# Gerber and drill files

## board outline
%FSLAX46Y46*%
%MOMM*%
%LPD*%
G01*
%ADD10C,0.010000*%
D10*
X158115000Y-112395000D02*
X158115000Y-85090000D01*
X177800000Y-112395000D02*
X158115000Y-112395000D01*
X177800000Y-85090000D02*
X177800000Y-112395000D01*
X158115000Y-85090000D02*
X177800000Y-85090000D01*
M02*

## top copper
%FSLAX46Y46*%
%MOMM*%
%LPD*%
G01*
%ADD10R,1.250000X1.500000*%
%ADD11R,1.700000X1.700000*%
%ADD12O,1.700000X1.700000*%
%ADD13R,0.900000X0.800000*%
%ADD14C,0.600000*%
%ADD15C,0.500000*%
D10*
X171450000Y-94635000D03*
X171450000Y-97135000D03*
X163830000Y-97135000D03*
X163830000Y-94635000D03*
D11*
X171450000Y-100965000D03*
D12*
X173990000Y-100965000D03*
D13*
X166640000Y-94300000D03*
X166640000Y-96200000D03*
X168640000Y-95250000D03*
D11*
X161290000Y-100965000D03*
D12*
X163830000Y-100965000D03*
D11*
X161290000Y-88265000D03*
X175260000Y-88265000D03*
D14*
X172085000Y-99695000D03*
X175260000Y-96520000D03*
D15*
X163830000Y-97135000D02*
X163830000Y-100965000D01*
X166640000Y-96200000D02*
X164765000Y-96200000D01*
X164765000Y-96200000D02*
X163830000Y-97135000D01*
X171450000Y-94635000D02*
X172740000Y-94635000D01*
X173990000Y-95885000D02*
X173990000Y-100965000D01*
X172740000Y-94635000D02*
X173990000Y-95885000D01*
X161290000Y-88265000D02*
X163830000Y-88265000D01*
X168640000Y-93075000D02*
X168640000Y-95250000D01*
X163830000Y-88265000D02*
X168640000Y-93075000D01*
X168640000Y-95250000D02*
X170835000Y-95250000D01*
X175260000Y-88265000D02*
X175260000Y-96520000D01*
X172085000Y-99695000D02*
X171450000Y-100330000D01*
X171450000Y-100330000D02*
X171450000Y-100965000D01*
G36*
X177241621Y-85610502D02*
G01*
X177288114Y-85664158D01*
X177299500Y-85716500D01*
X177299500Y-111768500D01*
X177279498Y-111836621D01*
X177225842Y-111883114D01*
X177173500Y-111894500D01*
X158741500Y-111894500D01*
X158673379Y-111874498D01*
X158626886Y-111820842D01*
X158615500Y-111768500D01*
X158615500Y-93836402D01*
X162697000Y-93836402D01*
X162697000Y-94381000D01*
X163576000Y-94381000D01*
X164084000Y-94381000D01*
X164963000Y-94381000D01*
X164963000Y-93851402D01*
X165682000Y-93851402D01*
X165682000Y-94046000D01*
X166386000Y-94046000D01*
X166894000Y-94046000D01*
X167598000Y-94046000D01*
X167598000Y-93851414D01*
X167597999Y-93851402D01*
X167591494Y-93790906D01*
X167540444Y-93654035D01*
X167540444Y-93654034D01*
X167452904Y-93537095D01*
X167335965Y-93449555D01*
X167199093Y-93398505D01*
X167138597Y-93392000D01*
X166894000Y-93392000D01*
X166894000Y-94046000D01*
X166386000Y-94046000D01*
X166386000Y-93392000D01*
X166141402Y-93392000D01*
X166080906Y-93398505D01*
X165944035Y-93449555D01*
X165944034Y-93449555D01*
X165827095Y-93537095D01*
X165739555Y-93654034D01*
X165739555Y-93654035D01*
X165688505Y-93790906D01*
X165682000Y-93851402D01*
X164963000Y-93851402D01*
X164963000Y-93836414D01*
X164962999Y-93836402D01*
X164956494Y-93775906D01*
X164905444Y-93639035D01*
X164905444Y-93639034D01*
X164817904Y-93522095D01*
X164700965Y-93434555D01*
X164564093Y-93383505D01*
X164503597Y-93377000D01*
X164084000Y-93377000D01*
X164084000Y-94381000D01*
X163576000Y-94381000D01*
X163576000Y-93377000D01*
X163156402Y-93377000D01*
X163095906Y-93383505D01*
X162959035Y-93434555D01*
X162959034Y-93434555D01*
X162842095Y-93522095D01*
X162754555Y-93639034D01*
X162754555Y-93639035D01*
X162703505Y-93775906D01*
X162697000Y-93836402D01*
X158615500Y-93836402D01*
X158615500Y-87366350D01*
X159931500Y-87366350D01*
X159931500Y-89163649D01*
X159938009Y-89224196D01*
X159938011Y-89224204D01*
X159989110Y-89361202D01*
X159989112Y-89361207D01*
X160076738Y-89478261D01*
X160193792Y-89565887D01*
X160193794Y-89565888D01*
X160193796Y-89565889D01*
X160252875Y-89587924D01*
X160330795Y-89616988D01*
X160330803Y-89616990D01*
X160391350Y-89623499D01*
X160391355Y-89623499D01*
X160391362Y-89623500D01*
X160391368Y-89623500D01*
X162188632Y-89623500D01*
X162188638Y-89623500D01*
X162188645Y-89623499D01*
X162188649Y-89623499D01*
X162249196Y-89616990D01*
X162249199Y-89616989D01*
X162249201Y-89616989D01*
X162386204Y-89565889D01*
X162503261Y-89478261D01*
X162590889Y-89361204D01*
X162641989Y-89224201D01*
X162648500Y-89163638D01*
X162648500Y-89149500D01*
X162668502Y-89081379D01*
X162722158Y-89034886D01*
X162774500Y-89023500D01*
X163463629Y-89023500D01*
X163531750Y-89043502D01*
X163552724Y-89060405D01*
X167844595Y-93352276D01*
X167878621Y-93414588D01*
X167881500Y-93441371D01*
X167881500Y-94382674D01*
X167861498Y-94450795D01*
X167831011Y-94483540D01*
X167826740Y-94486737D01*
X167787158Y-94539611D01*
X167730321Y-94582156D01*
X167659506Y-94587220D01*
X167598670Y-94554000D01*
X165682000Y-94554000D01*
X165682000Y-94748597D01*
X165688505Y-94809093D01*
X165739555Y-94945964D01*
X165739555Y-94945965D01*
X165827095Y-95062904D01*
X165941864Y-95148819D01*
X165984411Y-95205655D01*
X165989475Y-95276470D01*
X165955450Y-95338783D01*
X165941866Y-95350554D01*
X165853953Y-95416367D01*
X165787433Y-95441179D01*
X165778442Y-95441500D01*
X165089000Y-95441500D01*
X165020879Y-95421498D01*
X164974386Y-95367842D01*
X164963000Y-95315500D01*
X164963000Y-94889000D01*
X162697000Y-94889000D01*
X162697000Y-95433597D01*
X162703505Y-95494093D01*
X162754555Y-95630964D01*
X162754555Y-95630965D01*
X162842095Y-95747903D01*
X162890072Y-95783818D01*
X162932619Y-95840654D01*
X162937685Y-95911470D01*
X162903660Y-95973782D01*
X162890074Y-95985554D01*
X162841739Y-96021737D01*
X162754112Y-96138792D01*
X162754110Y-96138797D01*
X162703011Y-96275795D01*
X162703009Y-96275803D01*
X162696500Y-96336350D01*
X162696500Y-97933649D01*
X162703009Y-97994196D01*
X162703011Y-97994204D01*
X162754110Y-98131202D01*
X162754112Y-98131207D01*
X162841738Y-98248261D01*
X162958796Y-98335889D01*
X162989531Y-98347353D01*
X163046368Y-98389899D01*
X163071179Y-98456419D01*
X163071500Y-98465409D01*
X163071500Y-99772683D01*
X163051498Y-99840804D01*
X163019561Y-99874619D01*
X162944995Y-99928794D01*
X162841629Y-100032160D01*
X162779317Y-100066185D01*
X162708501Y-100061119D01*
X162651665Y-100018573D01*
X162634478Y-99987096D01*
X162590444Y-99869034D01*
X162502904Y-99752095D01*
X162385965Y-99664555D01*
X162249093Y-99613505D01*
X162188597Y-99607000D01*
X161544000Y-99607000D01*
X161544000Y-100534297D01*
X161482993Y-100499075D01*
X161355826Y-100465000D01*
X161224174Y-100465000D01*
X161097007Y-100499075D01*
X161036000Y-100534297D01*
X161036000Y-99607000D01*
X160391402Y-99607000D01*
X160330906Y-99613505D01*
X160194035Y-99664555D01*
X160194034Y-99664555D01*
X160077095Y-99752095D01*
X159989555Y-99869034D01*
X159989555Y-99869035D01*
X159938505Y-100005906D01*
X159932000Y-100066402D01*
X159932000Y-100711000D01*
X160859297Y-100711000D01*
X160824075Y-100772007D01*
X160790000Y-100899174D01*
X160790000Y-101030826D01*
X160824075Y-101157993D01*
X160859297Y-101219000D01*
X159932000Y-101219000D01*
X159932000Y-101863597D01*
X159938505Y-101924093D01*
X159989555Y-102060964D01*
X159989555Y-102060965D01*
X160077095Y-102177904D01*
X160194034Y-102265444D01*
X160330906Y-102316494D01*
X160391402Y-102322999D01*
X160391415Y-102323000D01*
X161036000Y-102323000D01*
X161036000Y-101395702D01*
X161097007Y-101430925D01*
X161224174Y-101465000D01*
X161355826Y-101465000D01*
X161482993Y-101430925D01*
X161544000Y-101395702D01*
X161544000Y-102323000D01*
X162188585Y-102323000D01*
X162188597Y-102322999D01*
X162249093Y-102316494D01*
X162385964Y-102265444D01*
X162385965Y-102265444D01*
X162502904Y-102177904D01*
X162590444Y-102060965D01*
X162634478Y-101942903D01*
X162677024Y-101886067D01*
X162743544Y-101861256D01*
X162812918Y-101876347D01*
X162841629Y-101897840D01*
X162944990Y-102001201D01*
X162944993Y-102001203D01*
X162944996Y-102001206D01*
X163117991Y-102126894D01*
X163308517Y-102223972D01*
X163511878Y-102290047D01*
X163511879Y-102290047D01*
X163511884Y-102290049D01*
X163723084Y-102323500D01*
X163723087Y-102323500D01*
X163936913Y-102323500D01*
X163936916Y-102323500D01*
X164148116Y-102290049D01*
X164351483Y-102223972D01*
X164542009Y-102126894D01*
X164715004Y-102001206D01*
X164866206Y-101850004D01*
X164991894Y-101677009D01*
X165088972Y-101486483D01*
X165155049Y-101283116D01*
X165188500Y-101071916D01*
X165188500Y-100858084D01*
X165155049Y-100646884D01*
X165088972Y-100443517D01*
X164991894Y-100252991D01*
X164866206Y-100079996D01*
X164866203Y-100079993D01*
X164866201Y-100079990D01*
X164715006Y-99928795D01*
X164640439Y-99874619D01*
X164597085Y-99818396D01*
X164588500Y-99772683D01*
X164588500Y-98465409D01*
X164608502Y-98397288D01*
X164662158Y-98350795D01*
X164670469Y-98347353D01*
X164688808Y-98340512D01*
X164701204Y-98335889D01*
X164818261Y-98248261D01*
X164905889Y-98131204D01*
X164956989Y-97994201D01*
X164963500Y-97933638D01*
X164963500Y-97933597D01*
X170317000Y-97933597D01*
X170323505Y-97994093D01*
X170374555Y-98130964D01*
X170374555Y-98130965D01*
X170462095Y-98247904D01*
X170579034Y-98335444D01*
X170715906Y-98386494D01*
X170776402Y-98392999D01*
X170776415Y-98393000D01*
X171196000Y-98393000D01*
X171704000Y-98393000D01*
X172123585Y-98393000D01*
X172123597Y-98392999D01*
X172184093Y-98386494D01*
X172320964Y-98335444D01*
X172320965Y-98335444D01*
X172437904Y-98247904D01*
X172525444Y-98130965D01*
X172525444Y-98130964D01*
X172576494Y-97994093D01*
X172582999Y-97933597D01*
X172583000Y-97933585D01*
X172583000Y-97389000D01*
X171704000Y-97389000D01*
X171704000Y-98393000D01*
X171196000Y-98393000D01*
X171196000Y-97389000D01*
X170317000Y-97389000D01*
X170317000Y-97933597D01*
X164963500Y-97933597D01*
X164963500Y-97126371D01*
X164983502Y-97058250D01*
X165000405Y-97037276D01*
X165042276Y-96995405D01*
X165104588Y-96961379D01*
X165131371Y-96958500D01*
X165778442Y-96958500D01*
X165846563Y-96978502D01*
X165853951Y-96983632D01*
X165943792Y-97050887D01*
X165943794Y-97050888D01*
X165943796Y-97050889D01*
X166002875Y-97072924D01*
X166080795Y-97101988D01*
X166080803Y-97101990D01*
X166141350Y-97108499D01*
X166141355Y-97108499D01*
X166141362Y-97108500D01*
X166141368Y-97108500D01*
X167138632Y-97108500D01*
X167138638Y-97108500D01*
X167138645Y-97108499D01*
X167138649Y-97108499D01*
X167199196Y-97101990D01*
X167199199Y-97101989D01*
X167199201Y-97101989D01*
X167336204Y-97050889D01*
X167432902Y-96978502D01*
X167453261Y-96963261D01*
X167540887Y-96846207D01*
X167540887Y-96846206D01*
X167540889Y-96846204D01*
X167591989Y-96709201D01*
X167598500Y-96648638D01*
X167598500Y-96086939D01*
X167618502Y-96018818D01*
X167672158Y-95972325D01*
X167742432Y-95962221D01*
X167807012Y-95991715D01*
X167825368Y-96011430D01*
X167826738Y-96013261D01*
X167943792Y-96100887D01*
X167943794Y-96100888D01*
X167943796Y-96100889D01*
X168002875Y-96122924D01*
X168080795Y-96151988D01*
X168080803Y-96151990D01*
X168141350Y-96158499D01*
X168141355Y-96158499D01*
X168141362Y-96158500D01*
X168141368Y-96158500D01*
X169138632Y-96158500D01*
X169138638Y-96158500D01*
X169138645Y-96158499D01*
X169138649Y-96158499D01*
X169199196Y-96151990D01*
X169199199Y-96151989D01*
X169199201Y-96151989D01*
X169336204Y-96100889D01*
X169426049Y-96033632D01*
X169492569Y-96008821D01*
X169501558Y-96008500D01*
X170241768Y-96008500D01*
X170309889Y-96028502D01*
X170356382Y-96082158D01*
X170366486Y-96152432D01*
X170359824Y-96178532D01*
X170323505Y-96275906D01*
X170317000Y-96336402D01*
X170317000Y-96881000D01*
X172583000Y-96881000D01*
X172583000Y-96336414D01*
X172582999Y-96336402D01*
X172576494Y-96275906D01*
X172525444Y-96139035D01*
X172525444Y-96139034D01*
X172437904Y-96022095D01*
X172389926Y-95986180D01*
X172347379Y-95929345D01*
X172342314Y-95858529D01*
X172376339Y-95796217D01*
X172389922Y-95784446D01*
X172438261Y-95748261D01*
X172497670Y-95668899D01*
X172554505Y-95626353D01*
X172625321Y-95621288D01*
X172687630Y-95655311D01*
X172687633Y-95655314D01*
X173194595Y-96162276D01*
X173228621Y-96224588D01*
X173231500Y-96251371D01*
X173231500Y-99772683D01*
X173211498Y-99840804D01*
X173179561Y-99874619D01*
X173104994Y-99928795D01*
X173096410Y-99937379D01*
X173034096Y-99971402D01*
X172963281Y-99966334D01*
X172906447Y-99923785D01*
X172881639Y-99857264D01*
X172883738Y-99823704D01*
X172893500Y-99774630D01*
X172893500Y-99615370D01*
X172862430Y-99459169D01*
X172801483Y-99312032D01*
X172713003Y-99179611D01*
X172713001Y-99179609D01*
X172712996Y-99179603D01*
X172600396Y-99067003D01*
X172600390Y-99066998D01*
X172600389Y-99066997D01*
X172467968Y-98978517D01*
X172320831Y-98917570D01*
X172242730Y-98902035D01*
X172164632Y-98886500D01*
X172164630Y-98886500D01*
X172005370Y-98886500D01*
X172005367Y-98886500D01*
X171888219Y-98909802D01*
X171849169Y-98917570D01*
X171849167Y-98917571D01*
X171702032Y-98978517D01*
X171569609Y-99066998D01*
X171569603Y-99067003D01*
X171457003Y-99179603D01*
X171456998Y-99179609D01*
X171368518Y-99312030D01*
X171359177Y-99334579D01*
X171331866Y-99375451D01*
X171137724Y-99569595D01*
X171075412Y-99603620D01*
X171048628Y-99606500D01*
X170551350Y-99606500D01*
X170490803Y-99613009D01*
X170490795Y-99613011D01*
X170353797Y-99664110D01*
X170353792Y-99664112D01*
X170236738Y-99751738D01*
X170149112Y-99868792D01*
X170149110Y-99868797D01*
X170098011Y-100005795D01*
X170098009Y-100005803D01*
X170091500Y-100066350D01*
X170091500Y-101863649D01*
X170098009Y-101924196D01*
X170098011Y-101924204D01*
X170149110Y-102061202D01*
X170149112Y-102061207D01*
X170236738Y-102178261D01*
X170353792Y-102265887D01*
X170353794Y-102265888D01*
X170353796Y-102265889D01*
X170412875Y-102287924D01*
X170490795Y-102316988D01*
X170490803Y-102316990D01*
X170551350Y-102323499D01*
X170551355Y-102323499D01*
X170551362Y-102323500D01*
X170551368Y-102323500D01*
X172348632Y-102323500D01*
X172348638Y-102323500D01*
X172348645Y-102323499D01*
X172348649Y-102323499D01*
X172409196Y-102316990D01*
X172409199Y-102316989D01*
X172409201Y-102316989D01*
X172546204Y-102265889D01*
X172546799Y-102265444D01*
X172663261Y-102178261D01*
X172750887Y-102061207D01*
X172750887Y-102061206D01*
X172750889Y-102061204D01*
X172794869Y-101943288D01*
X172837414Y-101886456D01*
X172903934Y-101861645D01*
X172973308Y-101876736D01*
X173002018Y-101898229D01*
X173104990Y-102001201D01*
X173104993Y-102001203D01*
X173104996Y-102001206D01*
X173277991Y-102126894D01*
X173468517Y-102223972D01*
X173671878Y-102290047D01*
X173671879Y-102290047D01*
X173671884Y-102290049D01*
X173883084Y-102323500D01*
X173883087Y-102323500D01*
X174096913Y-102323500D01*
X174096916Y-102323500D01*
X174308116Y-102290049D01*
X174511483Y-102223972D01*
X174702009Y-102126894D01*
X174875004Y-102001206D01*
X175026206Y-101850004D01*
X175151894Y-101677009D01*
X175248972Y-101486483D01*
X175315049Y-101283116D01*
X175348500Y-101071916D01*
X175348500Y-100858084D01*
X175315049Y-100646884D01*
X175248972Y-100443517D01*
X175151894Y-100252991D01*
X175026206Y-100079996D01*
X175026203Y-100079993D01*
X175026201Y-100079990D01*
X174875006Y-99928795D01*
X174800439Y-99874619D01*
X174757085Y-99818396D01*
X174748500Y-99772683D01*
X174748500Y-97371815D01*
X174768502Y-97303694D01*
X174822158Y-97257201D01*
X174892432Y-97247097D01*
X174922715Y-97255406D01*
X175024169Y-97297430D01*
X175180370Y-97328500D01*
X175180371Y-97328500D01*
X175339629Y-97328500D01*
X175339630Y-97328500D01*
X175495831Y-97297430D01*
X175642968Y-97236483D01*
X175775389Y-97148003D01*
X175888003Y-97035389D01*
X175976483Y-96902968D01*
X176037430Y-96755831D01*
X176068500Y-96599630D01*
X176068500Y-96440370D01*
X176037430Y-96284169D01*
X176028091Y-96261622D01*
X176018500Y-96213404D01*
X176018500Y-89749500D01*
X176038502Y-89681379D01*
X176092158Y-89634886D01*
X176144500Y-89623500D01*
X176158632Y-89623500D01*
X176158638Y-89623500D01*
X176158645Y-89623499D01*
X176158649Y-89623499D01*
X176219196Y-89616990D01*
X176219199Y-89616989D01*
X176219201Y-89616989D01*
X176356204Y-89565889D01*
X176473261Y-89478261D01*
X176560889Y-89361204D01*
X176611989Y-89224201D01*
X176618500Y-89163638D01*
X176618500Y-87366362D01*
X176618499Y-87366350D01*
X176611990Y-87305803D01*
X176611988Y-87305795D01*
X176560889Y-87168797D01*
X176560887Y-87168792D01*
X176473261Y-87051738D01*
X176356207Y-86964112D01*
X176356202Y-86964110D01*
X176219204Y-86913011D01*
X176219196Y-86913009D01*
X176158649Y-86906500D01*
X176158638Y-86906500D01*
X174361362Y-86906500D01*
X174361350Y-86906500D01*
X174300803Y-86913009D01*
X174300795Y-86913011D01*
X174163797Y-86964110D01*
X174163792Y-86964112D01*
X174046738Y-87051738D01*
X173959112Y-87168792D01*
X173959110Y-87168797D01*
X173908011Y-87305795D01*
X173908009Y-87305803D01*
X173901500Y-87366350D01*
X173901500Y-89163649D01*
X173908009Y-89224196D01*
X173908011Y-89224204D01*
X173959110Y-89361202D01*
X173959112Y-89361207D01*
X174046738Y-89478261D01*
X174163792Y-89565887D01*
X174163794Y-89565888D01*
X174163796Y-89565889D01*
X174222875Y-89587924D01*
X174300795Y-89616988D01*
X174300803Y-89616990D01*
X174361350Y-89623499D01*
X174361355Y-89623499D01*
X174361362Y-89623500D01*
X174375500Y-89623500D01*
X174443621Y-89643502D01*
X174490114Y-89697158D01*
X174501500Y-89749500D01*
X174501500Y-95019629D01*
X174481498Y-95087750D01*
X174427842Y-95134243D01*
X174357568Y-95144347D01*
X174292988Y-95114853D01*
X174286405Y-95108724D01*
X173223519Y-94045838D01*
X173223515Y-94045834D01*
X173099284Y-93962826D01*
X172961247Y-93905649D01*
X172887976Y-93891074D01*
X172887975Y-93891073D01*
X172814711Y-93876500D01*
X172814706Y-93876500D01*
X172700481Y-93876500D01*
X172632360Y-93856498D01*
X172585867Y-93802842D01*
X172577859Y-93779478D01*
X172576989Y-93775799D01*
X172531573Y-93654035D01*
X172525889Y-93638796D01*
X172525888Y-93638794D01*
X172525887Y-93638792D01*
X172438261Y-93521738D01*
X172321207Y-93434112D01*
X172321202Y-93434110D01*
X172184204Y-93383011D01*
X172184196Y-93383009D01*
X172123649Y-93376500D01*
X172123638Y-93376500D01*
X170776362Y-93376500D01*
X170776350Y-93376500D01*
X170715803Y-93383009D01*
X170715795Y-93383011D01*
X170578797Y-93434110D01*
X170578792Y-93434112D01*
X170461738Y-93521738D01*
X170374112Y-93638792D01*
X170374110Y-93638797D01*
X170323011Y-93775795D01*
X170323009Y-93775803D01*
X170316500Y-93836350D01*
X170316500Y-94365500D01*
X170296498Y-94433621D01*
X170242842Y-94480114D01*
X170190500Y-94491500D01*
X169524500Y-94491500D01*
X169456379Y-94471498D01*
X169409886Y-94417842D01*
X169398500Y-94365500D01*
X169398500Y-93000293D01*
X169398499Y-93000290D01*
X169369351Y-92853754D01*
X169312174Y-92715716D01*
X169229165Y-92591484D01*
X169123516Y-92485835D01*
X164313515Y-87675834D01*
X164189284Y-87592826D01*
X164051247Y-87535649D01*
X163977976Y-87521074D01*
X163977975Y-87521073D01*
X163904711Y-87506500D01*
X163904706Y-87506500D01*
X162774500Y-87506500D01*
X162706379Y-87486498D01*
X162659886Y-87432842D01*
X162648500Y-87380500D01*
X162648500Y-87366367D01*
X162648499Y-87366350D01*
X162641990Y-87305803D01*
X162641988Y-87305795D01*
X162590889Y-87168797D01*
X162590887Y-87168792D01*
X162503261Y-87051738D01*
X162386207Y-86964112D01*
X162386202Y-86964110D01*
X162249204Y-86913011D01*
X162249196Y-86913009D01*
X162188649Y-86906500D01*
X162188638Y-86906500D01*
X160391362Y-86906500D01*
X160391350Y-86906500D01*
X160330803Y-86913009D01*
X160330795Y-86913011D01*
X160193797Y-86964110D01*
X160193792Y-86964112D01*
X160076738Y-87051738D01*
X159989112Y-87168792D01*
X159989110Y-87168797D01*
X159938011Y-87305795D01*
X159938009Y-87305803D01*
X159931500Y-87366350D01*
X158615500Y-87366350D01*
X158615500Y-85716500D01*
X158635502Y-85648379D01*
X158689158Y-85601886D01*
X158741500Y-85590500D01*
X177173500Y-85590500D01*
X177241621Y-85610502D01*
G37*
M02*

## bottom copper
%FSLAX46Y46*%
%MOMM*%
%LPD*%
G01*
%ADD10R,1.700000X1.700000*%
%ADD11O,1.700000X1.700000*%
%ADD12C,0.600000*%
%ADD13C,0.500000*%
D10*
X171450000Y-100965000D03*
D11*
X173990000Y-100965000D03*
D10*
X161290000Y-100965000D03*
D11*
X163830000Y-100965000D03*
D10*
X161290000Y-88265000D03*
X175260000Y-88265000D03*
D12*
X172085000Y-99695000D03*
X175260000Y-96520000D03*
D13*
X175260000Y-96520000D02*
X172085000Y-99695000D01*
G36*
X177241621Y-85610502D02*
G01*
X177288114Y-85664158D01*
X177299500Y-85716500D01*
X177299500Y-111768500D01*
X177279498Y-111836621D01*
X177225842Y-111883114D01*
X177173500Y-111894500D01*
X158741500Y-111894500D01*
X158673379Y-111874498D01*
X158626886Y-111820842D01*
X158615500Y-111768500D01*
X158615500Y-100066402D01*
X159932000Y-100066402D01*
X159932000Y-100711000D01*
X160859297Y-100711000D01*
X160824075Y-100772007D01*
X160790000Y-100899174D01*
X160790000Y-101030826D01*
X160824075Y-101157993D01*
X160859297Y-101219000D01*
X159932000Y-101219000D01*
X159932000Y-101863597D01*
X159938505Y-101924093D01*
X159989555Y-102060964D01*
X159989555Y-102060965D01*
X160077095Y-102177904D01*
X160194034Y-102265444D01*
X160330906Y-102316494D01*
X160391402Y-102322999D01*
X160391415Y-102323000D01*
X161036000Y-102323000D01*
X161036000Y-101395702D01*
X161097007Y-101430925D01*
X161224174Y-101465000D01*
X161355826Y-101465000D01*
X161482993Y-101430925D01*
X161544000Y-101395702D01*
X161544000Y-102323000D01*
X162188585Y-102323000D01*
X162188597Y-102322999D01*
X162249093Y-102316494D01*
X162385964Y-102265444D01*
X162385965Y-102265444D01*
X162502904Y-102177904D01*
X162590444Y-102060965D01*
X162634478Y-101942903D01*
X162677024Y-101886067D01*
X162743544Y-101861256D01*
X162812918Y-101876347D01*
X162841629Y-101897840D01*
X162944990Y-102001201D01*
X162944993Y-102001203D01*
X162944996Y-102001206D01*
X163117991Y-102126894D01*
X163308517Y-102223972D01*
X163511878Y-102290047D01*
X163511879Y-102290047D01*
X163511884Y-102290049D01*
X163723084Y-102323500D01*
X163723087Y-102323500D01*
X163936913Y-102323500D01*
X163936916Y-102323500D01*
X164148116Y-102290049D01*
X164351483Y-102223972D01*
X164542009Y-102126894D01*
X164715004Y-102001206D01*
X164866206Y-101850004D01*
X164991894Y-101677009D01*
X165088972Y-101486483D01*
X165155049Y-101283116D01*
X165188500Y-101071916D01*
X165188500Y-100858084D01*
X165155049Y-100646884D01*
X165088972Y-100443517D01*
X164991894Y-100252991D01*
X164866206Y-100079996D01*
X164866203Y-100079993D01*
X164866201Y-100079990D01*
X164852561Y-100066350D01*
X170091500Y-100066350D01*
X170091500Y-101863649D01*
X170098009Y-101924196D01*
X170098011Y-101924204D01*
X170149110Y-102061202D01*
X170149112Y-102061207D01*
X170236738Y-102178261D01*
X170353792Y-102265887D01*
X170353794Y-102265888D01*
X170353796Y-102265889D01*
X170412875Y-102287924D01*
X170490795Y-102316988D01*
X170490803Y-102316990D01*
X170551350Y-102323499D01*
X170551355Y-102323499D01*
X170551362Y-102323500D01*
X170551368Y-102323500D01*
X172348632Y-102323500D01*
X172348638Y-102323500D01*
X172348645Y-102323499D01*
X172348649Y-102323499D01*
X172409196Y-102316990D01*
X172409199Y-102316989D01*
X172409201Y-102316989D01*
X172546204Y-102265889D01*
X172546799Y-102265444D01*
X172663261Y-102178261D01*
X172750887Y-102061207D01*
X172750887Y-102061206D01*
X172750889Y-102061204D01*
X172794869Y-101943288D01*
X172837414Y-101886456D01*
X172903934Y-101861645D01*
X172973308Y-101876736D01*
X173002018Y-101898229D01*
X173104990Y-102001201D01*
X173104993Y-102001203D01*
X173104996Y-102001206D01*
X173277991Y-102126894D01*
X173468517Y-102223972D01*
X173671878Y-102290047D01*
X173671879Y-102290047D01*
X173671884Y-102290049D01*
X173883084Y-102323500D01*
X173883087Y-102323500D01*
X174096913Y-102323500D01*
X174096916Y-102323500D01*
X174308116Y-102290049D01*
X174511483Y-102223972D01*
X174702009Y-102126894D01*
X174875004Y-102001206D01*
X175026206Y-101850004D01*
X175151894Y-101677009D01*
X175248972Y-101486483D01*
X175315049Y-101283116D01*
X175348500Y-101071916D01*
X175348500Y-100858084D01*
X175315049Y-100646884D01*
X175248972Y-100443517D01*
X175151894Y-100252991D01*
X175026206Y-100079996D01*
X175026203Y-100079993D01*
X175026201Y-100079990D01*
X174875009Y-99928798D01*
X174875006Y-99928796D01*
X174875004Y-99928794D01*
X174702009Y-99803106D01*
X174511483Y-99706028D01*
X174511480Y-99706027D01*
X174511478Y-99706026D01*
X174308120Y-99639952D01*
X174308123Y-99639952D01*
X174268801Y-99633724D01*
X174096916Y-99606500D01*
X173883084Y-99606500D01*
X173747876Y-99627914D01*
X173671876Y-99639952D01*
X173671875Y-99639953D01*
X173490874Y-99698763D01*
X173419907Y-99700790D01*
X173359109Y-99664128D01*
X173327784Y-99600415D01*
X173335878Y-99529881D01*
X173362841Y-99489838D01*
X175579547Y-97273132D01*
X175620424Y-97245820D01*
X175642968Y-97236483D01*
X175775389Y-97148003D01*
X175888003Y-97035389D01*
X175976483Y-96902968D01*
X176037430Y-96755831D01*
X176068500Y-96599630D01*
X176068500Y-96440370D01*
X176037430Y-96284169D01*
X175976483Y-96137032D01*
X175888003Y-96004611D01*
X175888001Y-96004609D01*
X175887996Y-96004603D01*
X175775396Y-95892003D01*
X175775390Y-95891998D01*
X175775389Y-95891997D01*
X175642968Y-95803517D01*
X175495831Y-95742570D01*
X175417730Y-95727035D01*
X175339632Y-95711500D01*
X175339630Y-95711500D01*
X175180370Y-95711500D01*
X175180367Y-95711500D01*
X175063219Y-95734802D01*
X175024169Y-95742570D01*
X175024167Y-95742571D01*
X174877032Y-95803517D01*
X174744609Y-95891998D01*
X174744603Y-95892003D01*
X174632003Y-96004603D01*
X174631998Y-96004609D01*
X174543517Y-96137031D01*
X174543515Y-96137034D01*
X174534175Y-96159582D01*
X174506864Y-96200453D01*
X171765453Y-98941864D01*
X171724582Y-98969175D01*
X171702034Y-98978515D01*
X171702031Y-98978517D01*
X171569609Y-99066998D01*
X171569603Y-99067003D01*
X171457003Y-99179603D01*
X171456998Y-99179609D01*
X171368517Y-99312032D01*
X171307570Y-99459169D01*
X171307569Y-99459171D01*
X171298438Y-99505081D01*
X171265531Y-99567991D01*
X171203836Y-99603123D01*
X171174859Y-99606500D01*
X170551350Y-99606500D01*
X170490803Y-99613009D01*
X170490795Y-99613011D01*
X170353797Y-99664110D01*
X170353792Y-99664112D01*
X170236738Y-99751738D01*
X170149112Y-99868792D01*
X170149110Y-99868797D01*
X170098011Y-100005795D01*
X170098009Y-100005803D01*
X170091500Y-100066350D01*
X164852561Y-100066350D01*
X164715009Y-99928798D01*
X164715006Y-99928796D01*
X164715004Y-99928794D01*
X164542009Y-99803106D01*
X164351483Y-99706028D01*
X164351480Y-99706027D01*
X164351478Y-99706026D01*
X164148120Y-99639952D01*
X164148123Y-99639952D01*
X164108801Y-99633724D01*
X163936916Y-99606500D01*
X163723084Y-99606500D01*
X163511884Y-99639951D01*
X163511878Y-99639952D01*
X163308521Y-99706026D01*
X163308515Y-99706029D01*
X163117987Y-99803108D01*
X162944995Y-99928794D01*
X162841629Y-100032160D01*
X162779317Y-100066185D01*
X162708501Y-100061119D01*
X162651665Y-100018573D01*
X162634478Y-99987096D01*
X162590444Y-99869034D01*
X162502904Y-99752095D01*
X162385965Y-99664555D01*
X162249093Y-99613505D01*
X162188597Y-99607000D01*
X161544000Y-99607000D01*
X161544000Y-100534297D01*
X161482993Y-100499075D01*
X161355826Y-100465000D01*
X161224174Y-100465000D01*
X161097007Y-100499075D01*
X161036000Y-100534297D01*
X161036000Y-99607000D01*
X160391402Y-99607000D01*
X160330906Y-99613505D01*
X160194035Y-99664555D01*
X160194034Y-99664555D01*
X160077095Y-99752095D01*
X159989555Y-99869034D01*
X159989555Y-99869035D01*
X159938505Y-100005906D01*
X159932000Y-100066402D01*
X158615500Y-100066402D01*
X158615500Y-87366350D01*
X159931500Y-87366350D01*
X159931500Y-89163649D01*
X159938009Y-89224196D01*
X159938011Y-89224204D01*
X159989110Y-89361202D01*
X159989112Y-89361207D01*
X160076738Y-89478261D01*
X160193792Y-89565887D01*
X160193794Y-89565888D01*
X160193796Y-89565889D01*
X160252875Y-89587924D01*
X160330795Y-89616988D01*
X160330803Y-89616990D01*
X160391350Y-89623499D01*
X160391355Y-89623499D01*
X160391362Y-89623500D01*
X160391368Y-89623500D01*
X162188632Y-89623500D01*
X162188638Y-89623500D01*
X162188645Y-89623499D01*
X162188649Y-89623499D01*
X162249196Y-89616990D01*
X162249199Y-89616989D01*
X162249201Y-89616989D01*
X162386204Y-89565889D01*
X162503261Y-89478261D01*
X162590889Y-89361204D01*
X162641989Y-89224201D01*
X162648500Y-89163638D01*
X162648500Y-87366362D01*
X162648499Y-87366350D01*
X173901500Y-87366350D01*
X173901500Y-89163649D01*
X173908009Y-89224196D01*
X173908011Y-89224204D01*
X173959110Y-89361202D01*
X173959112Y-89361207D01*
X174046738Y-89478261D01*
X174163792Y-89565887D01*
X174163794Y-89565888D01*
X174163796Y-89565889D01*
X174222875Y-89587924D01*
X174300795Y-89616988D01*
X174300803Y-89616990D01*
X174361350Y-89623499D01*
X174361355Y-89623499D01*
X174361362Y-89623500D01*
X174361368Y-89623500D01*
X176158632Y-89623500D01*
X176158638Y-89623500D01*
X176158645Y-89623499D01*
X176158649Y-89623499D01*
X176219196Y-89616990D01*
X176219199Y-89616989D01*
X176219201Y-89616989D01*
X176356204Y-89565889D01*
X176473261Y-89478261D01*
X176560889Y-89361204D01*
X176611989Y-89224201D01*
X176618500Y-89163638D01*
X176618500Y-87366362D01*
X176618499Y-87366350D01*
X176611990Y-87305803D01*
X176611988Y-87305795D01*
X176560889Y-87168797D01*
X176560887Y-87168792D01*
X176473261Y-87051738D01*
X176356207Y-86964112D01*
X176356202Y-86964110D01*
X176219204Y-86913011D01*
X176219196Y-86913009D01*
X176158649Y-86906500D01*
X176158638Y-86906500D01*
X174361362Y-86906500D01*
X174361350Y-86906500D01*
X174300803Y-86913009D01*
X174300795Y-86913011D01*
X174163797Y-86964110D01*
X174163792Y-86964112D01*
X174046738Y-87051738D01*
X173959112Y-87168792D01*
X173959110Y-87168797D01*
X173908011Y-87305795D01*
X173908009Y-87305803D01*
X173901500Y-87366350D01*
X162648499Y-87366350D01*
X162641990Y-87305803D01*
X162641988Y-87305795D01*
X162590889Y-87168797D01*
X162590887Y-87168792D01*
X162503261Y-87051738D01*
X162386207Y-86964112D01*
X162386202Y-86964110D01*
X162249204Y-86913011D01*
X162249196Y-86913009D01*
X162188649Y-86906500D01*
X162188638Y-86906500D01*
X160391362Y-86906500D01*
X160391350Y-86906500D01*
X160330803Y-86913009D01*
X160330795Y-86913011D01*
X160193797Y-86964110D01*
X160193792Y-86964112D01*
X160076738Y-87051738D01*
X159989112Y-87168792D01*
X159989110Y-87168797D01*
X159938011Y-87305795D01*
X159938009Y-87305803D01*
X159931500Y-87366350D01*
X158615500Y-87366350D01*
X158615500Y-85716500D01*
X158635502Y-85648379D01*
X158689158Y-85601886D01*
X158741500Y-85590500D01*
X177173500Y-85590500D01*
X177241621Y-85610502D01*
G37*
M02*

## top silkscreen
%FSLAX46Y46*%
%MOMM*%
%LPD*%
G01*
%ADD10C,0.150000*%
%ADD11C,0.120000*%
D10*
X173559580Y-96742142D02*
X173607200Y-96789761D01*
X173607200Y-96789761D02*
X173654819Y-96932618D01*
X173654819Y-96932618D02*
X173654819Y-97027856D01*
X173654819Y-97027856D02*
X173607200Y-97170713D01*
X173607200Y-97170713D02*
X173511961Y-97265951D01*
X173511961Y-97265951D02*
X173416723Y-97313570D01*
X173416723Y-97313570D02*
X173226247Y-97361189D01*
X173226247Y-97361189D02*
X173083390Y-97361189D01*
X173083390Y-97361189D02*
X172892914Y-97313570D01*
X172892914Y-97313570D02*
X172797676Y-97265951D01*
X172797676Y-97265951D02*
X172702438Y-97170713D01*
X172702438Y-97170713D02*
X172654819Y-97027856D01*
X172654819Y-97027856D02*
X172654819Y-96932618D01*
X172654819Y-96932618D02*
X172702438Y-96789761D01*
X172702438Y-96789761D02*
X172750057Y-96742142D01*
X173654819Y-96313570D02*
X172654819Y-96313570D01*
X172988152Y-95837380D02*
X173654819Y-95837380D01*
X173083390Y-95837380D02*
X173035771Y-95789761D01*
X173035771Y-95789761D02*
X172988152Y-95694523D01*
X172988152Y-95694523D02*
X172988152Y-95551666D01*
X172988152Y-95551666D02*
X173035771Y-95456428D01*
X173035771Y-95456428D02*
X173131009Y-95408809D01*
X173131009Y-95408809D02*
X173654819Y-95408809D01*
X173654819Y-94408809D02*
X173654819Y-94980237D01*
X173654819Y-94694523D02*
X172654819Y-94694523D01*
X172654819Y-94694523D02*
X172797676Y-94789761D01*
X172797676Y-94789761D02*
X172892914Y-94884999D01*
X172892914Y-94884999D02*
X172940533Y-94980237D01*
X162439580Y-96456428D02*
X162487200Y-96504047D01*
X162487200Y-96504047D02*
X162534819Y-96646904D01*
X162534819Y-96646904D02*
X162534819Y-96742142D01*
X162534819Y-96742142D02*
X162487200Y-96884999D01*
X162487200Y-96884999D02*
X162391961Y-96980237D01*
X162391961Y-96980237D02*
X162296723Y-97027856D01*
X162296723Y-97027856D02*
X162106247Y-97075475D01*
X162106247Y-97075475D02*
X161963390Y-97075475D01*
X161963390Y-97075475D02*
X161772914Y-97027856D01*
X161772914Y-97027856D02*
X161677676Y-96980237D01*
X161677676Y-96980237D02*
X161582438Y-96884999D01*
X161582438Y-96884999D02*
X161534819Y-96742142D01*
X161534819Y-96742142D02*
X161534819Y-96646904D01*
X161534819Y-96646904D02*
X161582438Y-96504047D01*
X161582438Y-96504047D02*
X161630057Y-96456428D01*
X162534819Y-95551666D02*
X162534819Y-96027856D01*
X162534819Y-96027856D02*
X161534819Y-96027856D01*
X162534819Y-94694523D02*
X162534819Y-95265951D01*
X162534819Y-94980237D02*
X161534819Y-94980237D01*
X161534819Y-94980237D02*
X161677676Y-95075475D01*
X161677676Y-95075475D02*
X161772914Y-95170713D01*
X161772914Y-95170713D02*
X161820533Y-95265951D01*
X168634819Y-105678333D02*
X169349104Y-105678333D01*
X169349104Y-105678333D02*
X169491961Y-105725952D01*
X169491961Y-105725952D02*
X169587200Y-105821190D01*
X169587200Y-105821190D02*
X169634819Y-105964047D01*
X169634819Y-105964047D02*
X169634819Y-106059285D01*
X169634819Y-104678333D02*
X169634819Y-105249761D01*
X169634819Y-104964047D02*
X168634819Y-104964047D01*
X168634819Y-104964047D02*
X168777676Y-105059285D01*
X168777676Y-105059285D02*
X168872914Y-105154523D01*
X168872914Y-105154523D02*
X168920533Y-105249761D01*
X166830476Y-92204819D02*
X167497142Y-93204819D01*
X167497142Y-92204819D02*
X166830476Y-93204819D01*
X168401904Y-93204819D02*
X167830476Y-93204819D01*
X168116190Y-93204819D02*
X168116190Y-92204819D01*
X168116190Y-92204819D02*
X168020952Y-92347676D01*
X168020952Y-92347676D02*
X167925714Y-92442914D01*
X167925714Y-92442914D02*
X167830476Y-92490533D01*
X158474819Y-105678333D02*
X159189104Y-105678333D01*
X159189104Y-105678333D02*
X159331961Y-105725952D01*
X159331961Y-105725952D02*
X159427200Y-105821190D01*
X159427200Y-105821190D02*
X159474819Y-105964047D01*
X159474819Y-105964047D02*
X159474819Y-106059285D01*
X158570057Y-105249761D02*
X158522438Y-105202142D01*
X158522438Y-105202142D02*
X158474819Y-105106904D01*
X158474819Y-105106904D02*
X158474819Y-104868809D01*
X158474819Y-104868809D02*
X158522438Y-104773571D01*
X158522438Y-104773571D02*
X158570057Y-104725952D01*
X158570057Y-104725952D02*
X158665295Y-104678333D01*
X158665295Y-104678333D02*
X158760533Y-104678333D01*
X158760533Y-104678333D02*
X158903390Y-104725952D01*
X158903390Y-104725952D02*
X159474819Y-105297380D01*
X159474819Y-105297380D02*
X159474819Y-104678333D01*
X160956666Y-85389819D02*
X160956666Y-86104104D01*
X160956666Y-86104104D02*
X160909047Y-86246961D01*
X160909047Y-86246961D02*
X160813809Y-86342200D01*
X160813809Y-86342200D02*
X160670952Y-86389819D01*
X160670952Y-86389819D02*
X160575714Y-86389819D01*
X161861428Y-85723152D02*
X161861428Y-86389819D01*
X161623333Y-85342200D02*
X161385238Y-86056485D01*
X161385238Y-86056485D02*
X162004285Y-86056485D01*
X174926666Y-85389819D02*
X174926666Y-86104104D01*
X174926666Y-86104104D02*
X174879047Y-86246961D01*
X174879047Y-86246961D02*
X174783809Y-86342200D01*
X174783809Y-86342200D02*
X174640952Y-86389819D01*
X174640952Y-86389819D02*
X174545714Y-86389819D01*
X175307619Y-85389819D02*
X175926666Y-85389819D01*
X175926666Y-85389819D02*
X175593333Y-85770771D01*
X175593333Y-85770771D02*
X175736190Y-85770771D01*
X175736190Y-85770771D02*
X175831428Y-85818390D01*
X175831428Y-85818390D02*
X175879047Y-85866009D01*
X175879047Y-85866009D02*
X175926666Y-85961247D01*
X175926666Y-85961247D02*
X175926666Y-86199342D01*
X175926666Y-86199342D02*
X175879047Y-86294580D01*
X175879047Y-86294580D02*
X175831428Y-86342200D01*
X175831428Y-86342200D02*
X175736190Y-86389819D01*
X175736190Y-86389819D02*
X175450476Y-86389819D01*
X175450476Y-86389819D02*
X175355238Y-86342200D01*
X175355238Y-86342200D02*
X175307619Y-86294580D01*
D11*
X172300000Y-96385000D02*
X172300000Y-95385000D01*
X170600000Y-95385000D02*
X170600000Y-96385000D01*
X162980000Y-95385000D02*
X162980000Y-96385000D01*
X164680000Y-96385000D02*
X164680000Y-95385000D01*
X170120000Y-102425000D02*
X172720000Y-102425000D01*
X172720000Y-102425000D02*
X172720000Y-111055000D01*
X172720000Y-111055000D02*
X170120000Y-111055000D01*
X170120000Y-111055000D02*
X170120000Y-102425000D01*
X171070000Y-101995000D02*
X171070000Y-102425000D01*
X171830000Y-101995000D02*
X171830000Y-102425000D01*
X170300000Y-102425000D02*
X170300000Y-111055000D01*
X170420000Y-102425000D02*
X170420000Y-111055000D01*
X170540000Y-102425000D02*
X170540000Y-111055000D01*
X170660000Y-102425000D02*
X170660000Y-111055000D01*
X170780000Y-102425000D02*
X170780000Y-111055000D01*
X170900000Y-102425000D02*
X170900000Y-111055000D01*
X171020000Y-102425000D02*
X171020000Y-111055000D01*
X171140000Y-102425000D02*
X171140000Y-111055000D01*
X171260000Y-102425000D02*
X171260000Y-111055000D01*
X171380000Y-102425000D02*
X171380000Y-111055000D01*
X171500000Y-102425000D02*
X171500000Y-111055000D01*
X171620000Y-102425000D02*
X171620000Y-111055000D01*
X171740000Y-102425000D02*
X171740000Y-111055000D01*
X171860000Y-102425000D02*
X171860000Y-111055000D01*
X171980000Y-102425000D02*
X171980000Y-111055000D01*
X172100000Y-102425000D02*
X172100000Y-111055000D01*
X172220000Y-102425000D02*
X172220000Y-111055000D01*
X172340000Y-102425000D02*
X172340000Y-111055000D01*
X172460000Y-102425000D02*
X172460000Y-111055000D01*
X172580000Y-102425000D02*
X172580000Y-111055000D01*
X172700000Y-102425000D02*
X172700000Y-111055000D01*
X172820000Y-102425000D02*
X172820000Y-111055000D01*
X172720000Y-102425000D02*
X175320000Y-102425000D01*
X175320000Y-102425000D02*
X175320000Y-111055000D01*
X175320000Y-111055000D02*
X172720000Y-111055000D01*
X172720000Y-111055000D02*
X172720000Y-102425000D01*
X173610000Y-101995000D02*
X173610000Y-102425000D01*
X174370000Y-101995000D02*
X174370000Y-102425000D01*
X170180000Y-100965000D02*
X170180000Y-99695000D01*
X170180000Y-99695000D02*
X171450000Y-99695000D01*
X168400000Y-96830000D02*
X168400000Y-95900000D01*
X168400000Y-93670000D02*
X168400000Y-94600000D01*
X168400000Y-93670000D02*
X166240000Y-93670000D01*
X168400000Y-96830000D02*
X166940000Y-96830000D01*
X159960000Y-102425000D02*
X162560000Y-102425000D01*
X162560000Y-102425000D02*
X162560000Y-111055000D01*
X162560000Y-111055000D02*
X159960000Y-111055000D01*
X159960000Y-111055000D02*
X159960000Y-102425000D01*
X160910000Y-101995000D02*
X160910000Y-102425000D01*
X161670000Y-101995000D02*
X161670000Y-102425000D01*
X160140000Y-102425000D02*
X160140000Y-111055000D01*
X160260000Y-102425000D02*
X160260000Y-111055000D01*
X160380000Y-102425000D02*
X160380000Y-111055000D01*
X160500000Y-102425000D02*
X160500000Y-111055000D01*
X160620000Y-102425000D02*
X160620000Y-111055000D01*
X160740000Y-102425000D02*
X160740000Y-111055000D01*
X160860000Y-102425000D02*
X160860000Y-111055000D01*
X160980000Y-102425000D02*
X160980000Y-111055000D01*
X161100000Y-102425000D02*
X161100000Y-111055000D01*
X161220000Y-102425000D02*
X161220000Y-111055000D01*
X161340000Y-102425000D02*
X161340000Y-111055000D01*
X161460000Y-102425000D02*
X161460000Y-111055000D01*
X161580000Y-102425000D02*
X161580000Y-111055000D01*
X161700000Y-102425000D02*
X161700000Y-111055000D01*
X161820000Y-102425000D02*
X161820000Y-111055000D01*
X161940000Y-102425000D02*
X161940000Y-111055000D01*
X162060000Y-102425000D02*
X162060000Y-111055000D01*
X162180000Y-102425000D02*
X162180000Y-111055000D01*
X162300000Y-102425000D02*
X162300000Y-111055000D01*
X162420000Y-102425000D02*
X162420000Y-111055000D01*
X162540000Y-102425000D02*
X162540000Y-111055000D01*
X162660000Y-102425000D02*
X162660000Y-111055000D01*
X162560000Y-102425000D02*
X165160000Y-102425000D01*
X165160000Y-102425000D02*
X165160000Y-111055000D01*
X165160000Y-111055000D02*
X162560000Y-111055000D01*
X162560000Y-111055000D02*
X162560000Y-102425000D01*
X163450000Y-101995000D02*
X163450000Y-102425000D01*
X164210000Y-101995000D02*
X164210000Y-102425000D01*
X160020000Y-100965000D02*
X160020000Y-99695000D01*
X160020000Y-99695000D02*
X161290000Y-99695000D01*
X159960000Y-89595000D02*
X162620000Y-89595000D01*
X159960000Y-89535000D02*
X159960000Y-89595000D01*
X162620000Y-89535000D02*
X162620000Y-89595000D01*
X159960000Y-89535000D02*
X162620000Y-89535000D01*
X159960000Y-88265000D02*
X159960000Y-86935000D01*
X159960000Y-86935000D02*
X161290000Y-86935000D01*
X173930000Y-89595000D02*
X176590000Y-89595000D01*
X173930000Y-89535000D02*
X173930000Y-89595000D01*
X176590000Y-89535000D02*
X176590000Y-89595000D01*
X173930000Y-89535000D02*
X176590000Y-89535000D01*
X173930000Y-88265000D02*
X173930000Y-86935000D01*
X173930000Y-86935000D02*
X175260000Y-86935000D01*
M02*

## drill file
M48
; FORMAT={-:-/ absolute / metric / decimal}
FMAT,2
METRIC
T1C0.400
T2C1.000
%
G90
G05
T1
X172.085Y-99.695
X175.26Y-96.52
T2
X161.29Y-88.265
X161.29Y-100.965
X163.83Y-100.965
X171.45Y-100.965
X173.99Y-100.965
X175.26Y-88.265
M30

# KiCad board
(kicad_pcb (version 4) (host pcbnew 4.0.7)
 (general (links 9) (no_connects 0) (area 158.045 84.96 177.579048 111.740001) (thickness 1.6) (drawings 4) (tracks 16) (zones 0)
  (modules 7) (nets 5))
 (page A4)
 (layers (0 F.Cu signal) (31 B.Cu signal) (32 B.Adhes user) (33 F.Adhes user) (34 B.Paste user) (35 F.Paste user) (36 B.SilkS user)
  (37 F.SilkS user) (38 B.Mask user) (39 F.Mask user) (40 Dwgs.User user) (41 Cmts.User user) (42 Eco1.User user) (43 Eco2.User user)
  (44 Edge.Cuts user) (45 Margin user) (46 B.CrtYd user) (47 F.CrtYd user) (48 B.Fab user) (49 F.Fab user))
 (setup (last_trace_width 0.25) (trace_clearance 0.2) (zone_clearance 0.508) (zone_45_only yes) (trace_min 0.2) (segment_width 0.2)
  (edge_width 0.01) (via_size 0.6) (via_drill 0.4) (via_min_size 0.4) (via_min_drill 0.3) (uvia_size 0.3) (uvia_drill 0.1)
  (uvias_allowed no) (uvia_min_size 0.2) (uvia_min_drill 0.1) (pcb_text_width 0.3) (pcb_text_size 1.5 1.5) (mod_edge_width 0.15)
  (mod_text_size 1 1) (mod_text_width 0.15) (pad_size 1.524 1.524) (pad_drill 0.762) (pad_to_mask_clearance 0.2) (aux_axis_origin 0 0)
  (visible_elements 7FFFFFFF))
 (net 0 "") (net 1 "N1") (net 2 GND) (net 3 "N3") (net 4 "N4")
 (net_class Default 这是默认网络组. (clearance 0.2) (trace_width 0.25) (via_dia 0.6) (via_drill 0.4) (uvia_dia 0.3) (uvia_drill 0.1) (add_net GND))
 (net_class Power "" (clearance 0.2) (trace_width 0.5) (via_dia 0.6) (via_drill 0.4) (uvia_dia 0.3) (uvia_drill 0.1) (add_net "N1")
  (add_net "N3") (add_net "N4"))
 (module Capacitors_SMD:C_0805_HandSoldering (layer F.Cu) (at 171.45 95.885 270)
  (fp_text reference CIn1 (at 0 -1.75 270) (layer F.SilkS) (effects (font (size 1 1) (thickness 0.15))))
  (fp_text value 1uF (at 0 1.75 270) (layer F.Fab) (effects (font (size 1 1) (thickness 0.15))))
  (fp_line (start 0.5 -0.85) (end -0.5 -0.85) (layer F.SilkS) (width 0.12))
  (fp_line (start -0.5 0.85) (end 0.5 0.85) (layer F.SilkS) (width 0.12))
  (pad 1 smd rect (at -1.25 0 270) (size 1.5 1.25) (layers F.Cu F.Paste F.Mask) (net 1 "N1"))
  (pad 2 smd rect (at 1.25 0 270) (size 1.5 1.25) (layers F.Cu F.Paste F.Mask) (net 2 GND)))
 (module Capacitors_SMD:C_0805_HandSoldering (layer F.Cu) (at 163.83 95.885 90)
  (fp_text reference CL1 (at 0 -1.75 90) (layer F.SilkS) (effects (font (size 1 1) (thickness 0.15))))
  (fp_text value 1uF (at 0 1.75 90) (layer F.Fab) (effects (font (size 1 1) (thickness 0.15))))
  (fp_line (start 0.5 -0.85) (end -0.5 -0.85) (layer F.SilkS) (width 0.12))
  (fp_line (start -0.5 0.85) (end 0.5 0.85) (layer F.SilkS) (width 0.12))
  (pad 1 smd rect (at -1.25 0 90) (size 1.5 1.25) (layers F.Cu F.Paste F.Mask) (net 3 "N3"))
  (pad 2 smd rect (at 1.25 0 90) (size 1.5 1.25) (layers F.Cu F.Paste F.Mask) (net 2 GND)))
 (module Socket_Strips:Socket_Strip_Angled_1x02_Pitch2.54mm (layer F.Cu) (at 171.45 100.965 90)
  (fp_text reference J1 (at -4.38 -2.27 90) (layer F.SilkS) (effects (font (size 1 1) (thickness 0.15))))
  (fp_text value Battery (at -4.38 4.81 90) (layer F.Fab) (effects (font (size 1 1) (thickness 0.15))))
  (fp_line (start -1.46 -1.33) (end -1.46 1.27) (layer F.SilkS) (width 0.12))
  (fp_line (start -1.46 1.27) (end -10.09 1.27) (layer F.SilkS) (width 0.12))
  (fp_line (start -10.09 1.27) (end -10.09 -1.33) (layer F.SilkS) (width 0.12))
  (fp_line (start -10.09 -1.33) (end -1.46 -1.33) (layer F.SilkS) (width 0.12))
  (fp_line (start -1.03 -0.38) (end -1.46 -0.38) (layer F.SilkS) (width 0.12))
  (fp_line (start -1.03 0.38) (end -1.46 0.38) (layer F.SilkS) (width 0.12))
  (fp_line (start -1.46 -1.15) (end -10.09 -1.15) (layer F.SilkS) (width 0.12))
  (fp_line (start -1.46 -1.03) (end -10.09 -1.03) (layer F.SilkS) (width 0.12))
  (fp_line (start -1.46 -0.91) (end -10.09 -0.91) (layer F.SilkS) (width 0.12))
  (fp_line (start -1.46 -0.79) (end -10.09 -0.79) (layer F.SilkS) (width 0.12))
  (fp_line (start -1.46 -0.67) (end -10.09 -0.67) (layer F.SilkS) (width 0.12))
  (fp_line (start -1.46 -0.55) (end -10.09 -0.55) (layer F.SilkS) (width 0.12))
  (fp_line (start -1.46 -0.43) (end -10.09 -0.43) (layer F.SilkS) (width 0.12))
  (fp_line (start -1.46 -0.31) (end -10.09 -0.31) (layer F.SilkS) (width 0.12))
  (fp_line (start -1.46 -0.19) (end -10.09 -0.19) (layer F.SilkS) (width 0.12))
  (fp_line (start -1.46 -0.07) (end -10.09 -0.07) (layer F.SilkS) (width 0.12))
  (fp_line (start -1.46 0.05) (end -10.09 0.05) (layer F.SilkS) (width 0.12))
  (fp_line (start -1.46 0.17) (end -10.09 0.17) (layer F.SilkS) (width 0.12))
  (fp_line (start -1.46 0.29) (end -10.09 0.29) (layer F.SilkS) (width 0.12))
  (fp_line (start -1.46 0.41) (end -10.09 0.41) (layer F.SilkS) (width 0.12))
  (fp_line (start -1.46 0.53) (end -10.09 0.53) (layer F.SilkS) (width 0.12))
  (fp_line (start -1.46 0.65) (end -10.09 0.65) (layer F.SilkS) (width 0.12))
  (fp_line (start -1.46 0.77) (end -10.09 0.77) (layer F.SilkS) (width 0.12))
  (fp_line (start -1.46 0.89) (end -10.09 0.89) (layer F.SilkS) (width 0.12))
  (fp_line (start -1.46 1.01) (end -10.09 1.01) (layer F.SilkS) (width 0.12))
  (fp_line (start -1.46 1.13) (end -10.09 1.13) (layer F.SilkS) (width 0.12))
  (fp_line (start -1.46 1.25) (end -10.09 1.25) (layer F.SilkS) (width 0.12))
  (fp_line (start -1.46 1.37) (end -10.09 1.37) (layer F.SilkS) (width 0.12))
  (fp_line (start -1.46 1.27) (end -1.46 3.87) (layer F.SilkS) (width 0.12))
  (fp_line (start -1.46 3.87) (end -10.09 3.87) (layer F.SilkS) (width 0.12))
  (fp_line (start -10.09 3.87) (end -10.09 1.27) (layer F.SilkS) (width 0.12))
  (fp_line (start -10.09 1.27) (end -1.46 1.27) (layer F.SilkS) (width 0.12))
  (fp_line (start -1.03 2.16) (end -1.46 2.16) (layer F.SilkS) (width 0.12))
  (fp_line (start -1.03 2.92) (end -1.46 2.92) (layer F.SilkS) (width 0.12))
  (fp_line (start 0 -1.27) (end 1.27 -1.27) (layer F.SilkS) (width 0.12))
  (fp_line (start 1.27 -1.27) (end 1.27 0) (layer F.SilkS) (width 0.12))
  (pad 1 thru_hole rect (at 0 0 90) (size 1.7 1.7) (drill 1) (layers *.Cu *.Mask) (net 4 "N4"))
  (pad 2 thru_hole oval (at 0 2.54 90) (size 1.7 1.7) (drill 1) (layers *.Cu *.Mask) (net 1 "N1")))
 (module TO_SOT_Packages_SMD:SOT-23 (layer F.Cu) (at 167.64 95.25)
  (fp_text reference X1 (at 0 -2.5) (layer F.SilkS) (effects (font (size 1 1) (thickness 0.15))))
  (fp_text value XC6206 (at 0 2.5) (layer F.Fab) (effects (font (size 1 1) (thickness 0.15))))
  (fp_line (start 0.76 1.58) (end 0.76 0.65) (layer F.SilkS) (width 0.12))
  (fp_line (start 0.76 -1.58) (end 0.76 -0.65) (layer F.SilkS) (width 0.12))
  (fp_line (start 0.76 -1.58) (end -1.4 -1.58) (layer F.SilkS) (width 0.12))
  (fp_line (start 0.76 1.58) (end -0.7 1.58) (layer F.SilkS) (width 0.12))
  (pad 1 smd rect (at -1 -0.95) (size 0.9 0.8) (layers F.Cu F.Paste F.Mask) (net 2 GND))
  (pad 2 smd rect (at -1 0.95) (size 0.9 0.8) (layers F.Cu F.Paste F.Mask) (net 3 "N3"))
  (pad 3 smd rect (at 1 0) (size 0.9 0.8) (layers F.Cu F.Paste F.Mask) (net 1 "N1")))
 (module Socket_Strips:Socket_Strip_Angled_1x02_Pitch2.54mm (layer F.Cu) (at 161.29 100.965 90)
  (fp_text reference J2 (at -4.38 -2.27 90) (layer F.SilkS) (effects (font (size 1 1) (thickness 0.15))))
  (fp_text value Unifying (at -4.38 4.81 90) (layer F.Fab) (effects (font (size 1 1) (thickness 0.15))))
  (fp_line (start -1.46 -1.33) (end -1.46 1.27) (layer F.SilkS) (width 0.12))
  (fp_line (start -1.46 1.27) (end -10.09 1.27) (layer F.SilkS) (width 0.12))
  (fp_line (start -10.09 1.27) (end -10.09 -1.33) (layer F.SilkS) (width 0.12))
  (fp_line (start -10.09 -1.33) (end -1.46 -1.33) (layer F.SilkS) (width 0.12))
  (fp_line (start -1.03 -0.38) (end -1.46 -0.38) (layer F.SilkS) (width 0.12))
  (fp_line (start -1.03 0.38) (end -1.46 0.38) (layer F.SilkS) (width 0.12))
  (fp_line (start -1.46 -1.15) (end -10.09 -1.15) (layer F.SilkS) (width 0.12))
  (fp_line (start -1.46 -1.03) (end -10.09 -1.03) (layer F.SilkS) (width 0.12))
  (fp_line (start -1.46 -0.91) (end -10.09 -0.91) (layer F.SilkS) (width 0.12))
  (fp_line (start -1.46 -0.79) (end -10.09 -0.79) (layer F.SilkS) (width 0.12))
  (fp_line (start -1.46 -0.67) (end -10.09 -0.67) (layer F.SilkS) (width 0.12))
  (fp_line (start -1.46 -0.55) (end -10.09 -0.55) (layer F.SilkS) (width 0.12))
  (fp_line (start -1.46 -0.43) (end -10.09 -0.43) (layer F.SilkS) (width 0.12))
  (fp_line (start -1.46 -0.31) (end -10.09 -0.31) (layer F.SilkS) (width 0.12))
  (fp_line (start -1.46 -0.19) (end -10.09 -0.19) (layer F.SilkS) (width 0.12))
  (fp_line (start -1.46 -0.07) (end -10.09 -0.07) (layer F.SilkS) (width 0.12))
  (fp_line (start -1.46 0.05) (end -10.09 0.05) (layer F.SilkS) (width 0.12))
  (fp_line (start -1.46 0.17) (end -10.09 0.17) (layer F.SilkS) (width 0.12))
  (fp_line (start -1.46 0.29) (end -10.09 0.29) (layer F.SilkS) (width 0.12))
  (fp_line (start -1.46 0.41) (end -10.09 0.41) (layer F.SilkS) (width 0.12))
  (fp_line (start -1.46 0.53) (end -10.09 0.53) (layer F.SilkS) (width 0.12))
  (fp_line (start -1.46 0.65) (end -10.09 0.65) (layer F.SilkS) (width 0.12))
  (fp_line (start -1.46 0.77) (end -10.09 0.77) (layer F.SilkS) (width 0.12))
  (fp_line (start -1.46 0.89) (end -10.09 0.89) (layer F.SilkS) (width 0.12))
  (fp_line (start -1.46 1.01) (end -10.09 1.01) (layer F.SilkS) (width 0.12))
  (fp_line (start -1.46 1.13) (end -10.09 1.13) (layer F.SilkS) (width 0.12))
  (fp_line (start -1.46 1.25) (end -10.09 1.25) (layer F.SilkS) (width 0.12))
  (fp_line (start -1.46 1.37) (end -10.09 1.37) (layer F.SilkS) (width 0.12))
  (fp_line (start -1.46 1.27) (end -1.46 3.87) (layer F.SilkS) (width 0.12))
  (fp_line (start -1.46 3.87) (end -10.09 3.87) (layer F.SilkS) (width 0.12))
  (fp_line (start -10.09 3.87) (end -10.09 1.27) (layer F.SilkS) (width 0.12))
  (fp_line (start -10.09 1.27) (end -1.46 1.27) (layer F.SilkS) (width 0.12))
  (fp_line (start -1.03 2.16) (end -1.46 2.16) (layer F.SilkS) (width 0.12))
  (fp_line (start -1.03 2.92) (end -1.46 2.92) (layer F.SilkS) (width 0.12))
  (fp_line (start 0 -1.27) (end 1.27 -1.27) (layer F.SilkS) (width 0.12))
  (fp_line (start 1.27 -1.27) (end 1.27 0) (layer F.SilkS) (width 0.12))
  (pad 1 thru_hole rect (at 0 0 90) (size 1.7 1.7) (drill 1) (layers *.Cu *.Mask) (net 2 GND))
  (pad 2 thru_hole oval (at 0 2.54 90) (size 1.7 1.7) (drill 1) (layers *.Cu *.Mask) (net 3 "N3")))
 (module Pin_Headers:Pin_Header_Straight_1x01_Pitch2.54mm (layer F.Cu) (at 161.29 88.265)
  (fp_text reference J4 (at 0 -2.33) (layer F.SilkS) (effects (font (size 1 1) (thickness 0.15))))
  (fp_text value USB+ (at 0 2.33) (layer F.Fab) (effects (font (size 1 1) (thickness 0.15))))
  (fp_line (start -1.33 1.33) (end 1.33 1.33) (layer F.SilkS) (width 0.12))
  (fp_line (start -1.33 1.27) (end -1.33 1.33) (layer F.SilkS) (width 0.12))
  (fp_line (start 1.33 1.27) (end 1.33 1.33) (layer F.SilkS) (width 0.12))
  (fp_line (start -1.33 1.27) (end 1.33 1.27) (layer F.SilkS) (width 0.12))
  (fp_line (start -1.33 0) (end -1.33 -1.33) (layer F.SilkS) (width 0.12))
  (fp_line (start -1.33 -1.33) (end 0 -1.33) (layer F.SilkS) (width 0.12))
  (pad 1 thru_hole rect (at 0 0) (size 1.7 1.7) (drill 1) (layers *.Cu *.Mask) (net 1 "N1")))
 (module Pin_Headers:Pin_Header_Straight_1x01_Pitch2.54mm (layer F.Cu) (at 175.26 88.265)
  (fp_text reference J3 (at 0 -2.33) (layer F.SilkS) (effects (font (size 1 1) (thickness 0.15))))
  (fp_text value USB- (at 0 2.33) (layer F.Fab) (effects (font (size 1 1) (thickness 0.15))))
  (fp_line (start -1.33 1.33) (end 1.33 1.33) (layer F.SilkS) (width 0.12))
  (fp_line (start -1.33 1.27) (end -1.33 1.33) (layer F.SilkS) (width 0.12))
  (fp_line (start 1.33 1.27) (end 1.33 1.33) (layer F.SilkS) (width 0.12))
  (fp_line (start -1.33 1.27) (end 1.33 1.27) (layer F.SilkS) (width 0.12))
  (fp_line (start -1.33 0) (end -1.33 -1.33) (layer F.SilkS) (width 0.12))
  (fp_line (start -1.33 -1.33) (end 0 -1.33) (layer F.SilkS) (width 0.12))
  (pad 1 thru_hole rect (at 0 0) (size 1.7 1.7) (drill 1) (layers *.Cu *.Mask) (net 4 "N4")))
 (gr_line (start 158.115 112.395) (end 158.115 85.09) (angle 90) (layer Edge.Cuts) (width 0.01))
 (gr_line (start 177.8 112.395) (end 158.115 112.395) (angle 90) (layer Edge.Cuts) (width 0.01))
 (gr_line (start 177.8 85.09) (end 177.8 112.395) (angle 90) (layer Edge.Cuts) (width 0.01))
 (gr_line (start 158.115 85.09) (end 177.8 85.09) (angle 90) (layer Edge.Cuts) (width 0.01))
 (segment (start 163.83 97.135) (end 163.83 100.965) (width 0.5) (layer F.Cu) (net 3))
 (segment (start 166.64 96.2) (end 164.765 96.2) (width 0.5) (layer F.Cu) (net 3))
 (segment (start 164.765 96.2) (end 163.83 97.135) (width 0.5) (layer F.Cu) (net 3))
 (segment (start 171.45 94.635) (end 172.74 94.635) (width 0.5) (layer F.Cu) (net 1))
 (segment (start 173.99 95.885) (end 173.99 100.965) (width 0.5) (layer F.Cu) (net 1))
 (segment (start 172.74 94.635) (end 173.99 95.885) (width 0.5) (layer F.Cu) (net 1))
 (segment (start 161.29 88.265) (end 163.83 88.265) (width 0.5) (layer F.Cu) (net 1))
 (segment (start 168.64 93.075) (end 168.64 95.25) (width 0.5) (layer F.Cu) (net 1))
 (segment (start 163.83 88.265) (end 168.64 93.075) (width 0.5) (layer F.Cu) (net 1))
 (segment (start 168.64 95.25) (end 170.835 95.25) (width 0.5) (layer F.Cu) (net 1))
 (segment (start 175.26 88.265) (end 175.26 96.52) (width 0.5) (layer F.Cu) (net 4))
 (segment (start 172.085 99.695) (end 171.45 100.33) (width 0.5) (layer F.Cu) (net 4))
 (via (at 172.085 99.695) (size 0.6) (drill 0.4) (layers F.Cu B.Cu) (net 4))
 (segment (start 175.26 96.52) (end 172.085 99.695) (width 0.5) (layer B.Cu) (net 4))
 (via (at 175.26 96.52) (size 0.6) (drill 0.4) (layers F.Cu B.Cu) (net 4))
 (segment (start 171.45 100.33) (end 171.45 100.965) (width 0.5) (layer F.Cu) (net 4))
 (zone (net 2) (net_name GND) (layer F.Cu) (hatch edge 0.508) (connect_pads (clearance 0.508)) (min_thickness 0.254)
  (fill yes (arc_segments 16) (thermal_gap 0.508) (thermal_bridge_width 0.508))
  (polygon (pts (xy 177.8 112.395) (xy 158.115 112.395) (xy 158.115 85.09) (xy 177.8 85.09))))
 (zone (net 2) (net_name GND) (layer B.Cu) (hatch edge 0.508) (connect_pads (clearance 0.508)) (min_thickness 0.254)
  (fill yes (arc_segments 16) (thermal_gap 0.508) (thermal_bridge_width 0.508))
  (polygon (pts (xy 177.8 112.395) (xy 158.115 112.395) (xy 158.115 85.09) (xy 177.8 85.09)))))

